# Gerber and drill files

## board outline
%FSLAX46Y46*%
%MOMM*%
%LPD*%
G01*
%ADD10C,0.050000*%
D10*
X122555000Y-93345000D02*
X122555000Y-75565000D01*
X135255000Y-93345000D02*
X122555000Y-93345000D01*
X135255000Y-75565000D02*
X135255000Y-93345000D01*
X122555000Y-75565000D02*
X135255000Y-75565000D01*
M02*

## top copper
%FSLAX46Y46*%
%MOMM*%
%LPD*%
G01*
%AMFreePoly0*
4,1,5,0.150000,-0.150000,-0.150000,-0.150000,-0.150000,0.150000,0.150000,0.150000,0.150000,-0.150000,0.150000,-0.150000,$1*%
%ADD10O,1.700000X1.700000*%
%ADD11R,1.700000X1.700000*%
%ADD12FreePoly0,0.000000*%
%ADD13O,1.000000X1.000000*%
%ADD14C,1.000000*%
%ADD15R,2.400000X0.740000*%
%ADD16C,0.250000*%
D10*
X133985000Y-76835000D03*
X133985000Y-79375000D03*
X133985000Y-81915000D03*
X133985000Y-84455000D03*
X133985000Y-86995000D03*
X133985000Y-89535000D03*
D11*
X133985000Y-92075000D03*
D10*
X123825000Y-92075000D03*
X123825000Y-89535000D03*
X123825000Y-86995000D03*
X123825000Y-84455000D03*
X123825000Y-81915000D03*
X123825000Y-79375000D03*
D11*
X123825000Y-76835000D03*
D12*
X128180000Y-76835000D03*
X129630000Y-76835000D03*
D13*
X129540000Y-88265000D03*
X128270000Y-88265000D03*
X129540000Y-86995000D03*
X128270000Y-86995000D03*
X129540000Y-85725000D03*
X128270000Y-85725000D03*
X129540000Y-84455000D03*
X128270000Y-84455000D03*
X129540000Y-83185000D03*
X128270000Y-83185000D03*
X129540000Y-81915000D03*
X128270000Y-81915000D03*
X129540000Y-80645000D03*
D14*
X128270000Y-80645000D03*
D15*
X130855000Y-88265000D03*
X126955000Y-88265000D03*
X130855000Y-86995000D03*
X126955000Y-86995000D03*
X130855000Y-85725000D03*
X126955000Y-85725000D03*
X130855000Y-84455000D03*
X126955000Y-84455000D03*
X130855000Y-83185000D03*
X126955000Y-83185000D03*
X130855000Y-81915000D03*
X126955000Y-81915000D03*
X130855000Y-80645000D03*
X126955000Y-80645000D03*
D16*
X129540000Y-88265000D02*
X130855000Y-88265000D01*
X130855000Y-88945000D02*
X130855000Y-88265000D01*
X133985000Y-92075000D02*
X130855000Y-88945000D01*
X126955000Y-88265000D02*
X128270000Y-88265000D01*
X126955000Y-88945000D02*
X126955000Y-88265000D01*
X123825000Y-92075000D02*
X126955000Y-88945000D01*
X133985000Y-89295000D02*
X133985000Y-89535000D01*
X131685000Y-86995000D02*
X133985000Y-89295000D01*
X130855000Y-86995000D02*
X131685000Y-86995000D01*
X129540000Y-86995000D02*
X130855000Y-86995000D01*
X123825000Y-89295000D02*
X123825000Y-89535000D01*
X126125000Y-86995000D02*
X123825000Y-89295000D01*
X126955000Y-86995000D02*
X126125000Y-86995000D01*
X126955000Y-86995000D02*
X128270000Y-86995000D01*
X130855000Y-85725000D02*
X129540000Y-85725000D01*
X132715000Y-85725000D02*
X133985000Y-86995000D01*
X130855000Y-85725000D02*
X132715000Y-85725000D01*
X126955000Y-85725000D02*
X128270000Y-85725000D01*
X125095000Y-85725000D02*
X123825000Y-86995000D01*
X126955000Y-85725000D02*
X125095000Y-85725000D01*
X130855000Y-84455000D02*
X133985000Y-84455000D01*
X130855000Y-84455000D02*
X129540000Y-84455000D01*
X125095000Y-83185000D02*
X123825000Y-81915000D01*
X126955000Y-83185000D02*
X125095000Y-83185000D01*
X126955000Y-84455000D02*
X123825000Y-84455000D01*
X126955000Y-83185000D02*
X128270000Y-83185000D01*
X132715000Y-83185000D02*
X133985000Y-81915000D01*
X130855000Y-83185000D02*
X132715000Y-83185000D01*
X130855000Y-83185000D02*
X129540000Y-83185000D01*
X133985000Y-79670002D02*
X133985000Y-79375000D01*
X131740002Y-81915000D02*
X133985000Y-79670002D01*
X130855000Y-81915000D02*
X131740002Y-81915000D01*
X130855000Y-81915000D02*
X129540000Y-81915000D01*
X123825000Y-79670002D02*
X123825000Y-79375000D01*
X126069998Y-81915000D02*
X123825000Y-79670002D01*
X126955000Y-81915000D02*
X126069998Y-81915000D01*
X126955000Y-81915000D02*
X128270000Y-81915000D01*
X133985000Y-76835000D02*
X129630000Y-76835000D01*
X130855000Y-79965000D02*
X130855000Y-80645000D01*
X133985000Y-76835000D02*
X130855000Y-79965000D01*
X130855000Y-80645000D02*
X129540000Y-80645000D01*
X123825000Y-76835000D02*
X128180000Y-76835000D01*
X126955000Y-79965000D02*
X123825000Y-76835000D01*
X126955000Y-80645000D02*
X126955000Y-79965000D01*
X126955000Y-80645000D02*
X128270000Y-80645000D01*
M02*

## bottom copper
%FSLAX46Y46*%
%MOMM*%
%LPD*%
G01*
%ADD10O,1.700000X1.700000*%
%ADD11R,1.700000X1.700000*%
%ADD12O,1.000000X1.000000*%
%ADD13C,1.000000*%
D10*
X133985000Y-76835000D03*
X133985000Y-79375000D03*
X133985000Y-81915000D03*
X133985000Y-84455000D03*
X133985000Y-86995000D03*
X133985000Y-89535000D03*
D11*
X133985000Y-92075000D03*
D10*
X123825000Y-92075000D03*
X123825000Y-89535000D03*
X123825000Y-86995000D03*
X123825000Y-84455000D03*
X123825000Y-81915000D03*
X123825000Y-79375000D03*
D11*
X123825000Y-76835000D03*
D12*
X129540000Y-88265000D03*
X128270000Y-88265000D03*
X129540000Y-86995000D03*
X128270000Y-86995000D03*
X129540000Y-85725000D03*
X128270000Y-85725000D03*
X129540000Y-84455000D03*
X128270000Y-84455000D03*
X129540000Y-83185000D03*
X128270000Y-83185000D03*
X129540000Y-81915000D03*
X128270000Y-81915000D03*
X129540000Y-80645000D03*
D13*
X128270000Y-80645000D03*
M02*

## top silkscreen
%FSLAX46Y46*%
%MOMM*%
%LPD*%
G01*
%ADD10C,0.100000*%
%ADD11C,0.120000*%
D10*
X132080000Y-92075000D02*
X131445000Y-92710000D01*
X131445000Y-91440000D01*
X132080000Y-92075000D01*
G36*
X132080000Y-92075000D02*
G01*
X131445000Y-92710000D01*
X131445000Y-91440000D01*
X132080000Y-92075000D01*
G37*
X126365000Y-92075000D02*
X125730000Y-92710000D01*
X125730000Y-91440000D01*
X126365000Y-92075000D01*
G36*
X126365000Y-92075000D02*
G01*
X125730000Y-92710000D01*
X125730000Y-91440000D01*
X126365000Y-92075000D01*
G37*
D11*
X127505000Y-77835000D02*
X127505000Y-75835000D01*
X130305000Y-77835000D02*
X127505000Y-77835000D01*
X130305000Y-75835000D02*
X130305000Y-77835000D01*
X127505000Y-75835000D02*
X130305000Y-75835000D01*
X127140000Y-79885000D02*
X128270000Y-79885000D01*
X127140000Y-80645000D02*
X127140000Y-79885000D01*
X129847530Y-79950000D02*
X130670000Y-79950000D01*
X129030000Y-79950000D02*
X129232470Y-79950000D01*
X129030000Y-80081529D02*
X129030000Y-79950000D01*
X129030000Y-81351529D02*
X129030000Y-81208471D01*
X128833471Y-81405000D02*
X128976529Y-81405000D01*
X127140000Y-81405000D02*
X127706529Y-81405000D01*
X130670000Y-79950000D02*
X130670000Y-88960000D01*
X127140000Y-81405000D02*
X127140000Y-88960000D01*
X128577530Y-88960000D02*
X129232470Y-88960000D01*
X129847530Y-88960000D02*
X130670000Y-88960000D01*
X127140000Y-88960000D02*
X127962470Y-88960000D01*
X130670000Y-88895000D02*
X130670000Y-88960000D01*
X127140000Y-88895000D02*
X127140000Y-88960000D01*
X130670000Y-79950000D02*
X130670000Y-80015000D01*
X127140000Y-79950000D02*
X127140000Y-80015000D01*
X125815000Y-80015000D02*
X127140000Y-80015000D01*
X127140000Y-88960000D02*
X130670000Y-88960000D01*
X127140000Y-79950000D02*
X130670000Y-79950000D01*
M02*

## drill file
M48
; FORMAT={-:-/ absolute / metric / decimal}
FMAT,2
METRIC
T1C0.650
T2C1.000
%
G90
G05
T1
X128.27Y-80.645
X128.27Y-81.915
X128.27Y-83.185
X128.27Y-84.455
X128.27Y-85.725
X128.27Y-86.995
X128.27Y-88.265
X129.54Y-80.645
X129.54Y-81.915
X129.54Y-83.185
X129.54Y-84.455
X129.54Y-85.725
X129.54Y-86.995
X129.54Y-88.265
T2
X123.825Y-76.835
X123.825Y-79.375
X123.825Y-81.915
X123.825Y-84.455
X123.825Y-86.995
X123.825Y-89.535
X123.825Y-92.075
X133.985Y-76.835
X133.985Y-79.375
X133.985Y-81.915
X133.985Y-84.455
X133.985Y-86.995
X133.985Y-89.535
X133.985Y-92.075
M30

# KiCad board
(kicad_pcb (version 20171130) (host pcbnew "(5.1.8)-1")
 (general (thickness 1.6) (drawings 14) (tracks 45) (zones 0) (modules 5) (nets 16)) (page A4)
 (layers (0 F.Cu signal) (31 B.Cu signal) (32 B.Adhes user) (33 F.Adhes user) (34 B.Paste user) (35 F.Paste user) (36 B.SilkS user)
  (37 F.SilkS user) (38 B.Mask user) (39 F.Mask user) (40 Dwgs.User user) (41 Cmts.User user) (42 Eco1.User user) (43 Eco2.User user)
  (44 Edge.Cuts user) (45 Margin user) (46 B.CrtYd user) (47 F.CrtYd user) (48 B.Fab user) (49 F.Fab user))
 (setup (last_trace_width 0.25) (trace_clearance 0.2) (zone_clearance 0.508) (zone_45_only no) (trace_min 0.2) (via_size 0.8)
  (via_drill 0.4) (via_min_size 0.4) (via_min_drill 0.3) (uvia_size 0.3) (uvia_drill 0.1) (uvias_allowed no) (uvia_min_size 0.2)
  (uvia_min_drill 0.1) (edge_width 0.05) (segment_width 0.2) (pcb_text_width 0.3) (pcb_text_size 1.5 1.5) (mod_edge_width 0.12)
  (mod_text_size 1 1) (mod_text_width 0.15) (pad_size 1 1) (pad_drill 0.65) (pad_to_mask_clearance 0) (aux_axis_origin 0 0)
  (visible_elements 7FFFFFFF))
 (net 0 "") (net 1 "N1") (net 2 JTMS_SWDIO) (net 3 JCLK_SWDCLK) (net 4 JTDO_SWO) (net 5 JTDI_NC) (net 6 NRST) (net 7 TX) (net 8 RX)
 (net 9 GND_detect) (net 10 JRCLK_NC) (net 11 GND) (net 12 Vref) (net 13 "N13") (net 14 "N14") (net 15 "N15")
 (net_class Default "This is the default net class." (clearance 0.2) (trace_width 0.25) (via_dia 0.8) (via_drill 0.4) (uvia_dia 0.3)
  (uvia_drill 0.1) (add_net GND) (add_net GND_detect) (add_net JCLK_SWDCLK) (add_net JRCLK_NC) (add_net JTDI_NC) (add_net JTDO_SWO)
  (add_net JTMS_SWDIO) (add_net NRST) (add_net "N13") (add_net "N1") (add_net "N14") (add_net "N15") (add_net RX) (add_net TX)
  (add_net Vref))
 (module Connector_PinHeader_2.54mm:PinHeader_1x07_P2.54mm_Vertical (layer B.Cu) (at 133.985 92.075)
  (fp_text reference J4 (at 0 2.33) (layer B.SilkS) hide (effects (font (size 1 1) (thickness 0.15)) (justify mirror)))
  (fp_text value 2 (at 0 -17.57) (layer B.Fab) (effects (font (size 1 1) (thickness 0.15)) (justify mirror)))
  (pad 7 thru_hole oval (at 0 -15.24) (size 1.7 1.7) (drill 1) (layers *.Cu *.Mask) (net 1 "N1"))
  (pad 6 thru_hole oval (at 0 -12.7) (size 1.7 1.7) (drill 1) (layers *.Cu *.Mask) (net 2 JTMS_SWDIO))
  (pad 5 thru_hole oval (at 0 -10.16) (size 1.7 1.7) (drill 1) (layers *.Cu *.Mask) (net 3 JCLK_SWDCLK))
  (pad 4 thru_hole oval (at 0 -7.62) (size 1.7 1.7) (drill 1) (layers *.Cu *.Mask) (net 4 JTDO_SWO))
  (pad 3 thru_hole oval (at 0 -5.08) (size 1.7 1.7) (drill 1) (layers *.Cu *.Mask) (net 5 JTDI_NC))
  (pad 2 thru_hole oval (at 0 -2.54) (size 1.7 1.7) (drill 1) (layers *.Cu *.Mask) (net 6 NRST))
  (pad 1 thru_hole rect (at 0 0) (size 1.7 1.7) (drill 1) (layers *.Cu *.Mask) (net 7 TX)))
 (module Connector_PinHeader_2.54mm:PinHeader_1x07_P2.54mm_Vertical (layer B.Cu) (at 123.825 76.835 180)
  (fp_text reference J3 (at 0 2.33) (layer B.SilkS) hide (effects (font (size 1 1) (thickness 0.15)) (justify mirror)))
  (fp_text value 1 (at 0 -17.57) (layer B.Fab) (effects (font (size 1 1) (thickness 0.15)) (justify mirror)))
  (pad 7 thru_hole oval (at 0 -15.24 180) (size 1.7 1.7) (drill 1) (layers *.Cu *.Mask) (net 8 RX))
  (pad 6 thru_hole oval (at 0 -12.7 180) (size 1.7 1.7) (drill 1) (layers *.Cu *.Mask) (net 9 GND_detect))
  (pad 5 thru_hole oval (at 0 -10.16 180) (size 1.7 1.7) (drill 1) (layers *.Cu *.Mask) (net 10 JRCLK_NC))
  (pad 4 thru_hole oval (at 0 -7.62 180) (size 1.7 1.7) (drill 1) (layers *.Cu *.Mask) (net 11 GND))
  (pad 3 thru_hole oval (at 0 -5.08 180) (size 1.7 1.7) (drill 1) (layers *.Cu *.Mask) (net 11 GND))
  (pad 2 thru_hole oval (at 0 -2.54 180) (size 1.7 1.7) (drill 1) (layers *.Cu *.Mask) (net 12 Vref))
  (pad 1 thru_hole rect (at 0 0 180) (size 1.7 1.7) (drill 1) (layers *.Cu *.Mask) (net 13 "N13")))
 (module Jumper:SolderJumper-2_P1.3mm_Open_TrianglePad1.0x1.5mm (layer F.Cu) (at 128.905 76.835)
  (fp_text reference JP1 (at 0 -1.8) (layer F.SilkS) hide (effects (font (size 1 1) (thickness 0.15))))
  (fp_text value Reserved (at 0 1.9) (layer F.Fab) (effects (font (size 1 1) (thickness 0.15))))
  (fp_line (start -1.4 1) (end -1.4 -1) (layer F.SilkS) (width 0.12))
  (fp_line (start 1.4 1) (end -1.4 1) (layer F.SilkS) (width 0.12))
  (fp_line (start 1.4 -1) (end 1.4 1) (layer F.SilkS) (width 0.12))
  (fp_line (start -1.4 -1) (end 1.4 -1) (layer F.SilkS) (width 0.12))
  (pad 1 smd custom (at -0.725 0) (size 0.3 0.3) (layers F.Cu F.Mask) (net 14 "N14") (zone_connect 2)
   (options (clearance outline) (anchor rect)) (primitives))
  (pad 2 smd custom (at 0.725 0) (size 0.3 0.3) (layers F.Cu F.Mask) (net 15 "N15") (zone_connect 2)
   (options (clearance outline) (anchor rect)) (primitives)))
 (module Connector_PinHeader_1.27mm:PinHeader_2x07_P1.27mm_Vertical (layer F.Cu) (at 128.27 80.645)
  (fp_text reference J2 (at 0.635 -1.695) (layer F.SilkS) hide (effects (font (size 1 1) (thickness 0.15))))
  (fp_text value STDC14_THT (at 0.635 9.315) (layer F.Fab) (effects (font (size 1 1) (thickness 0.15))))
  (fp_line (start -1.13 -0.76) (end 0 -0.76) (layer F.SilkS) (width 0.12))
  (fp_line (start -1.13 0) (end -1.13 -0.76) (layer F.SilkS) (width 0.12))
  (fp_line (start 1.57753 -0.695) (end 2.4 -0.695) (layer F.SilkS) (width 0.12))
  (fp_line (start 0.76 -0.695) (end 0.96247 -0.695) (layer F.SilkS) (width 0.12))
  (fp_line (start 0.76 -0.563471) (end 0.76 -0.695) (layer F.SilkS) (width 0.12))
  (fp_line (start 0.76 0.706529) (end 0.76 0.563471) (layer F.SilkS) (width 0.12))
  (fp_line (start 0.563471 0.76) (end 0.706529 0.76) (layer F.SilkS) (width 0.12))
  (fp_line (start -1.13 0.76) (end -0.563471 0.76) (layer F.SilkS) (width 0.12))
  (fp_line (start 2.4 -0.695) (end 2.4 8.315) (layer F.SilkS) (width 0.12))
  (fp_line (start -1.13 0.76) (end -1.13 8.315) (layer F.SilkS) (width 0.12))
  (fp_line (start 0.30753 8.315) (end 0.96247 8.315) (layer F.SilkS) (width 0.12))
  (fp_line (start 1.57753 8.315) (end 2.4 8.315) (layer F.SilkS) (width 0.12))
  (fp_line (start -1.13 8.315) (end -0.30753 8.315) (layer F.SilkS) (width 0.12))
  (pad 14 thru_hole oval (at 1.27 7.62) (size 1 1) (drill 0.65) (layers *.Cu *.Mask) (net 7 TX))
  (pad 13 thru_hole oval (at 0 7.62) (size 1 1) (drill 0.65) (layers *.Cu *.Mask) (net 8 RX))
  (pad 12 thru_hole oval (at 1.27 6.35) (size 1 1) (drill 0.65) (layers *.Cu *.Mask) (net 6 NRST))
  (pad 11 thru_hole oval (at 0 6.35) (size 1 1) (drill 0.65) (layers *.Cu *.Mask) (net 9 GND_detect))
  (pad 10 thru_hole oval (at 1.27 5.08) (size 1 1) (drill 0.65) (layers *.Cu *.Mask) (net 5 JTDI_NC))
  (pad 9 thru_hole oval (at 0 5.08) (size 1 1) (drill 0.65) (layers *.Cu *.Mask) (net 10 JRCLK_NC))
  (pad 8 thru_hole oval (at 1.27 3.81) (size 1 1) (drill 0.65) (layers *.Cu *.Mask) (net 4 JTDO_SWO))
  (pad 7 thru_hole oval (at 0 3.81) (size 1 1) (drill 0.65) (layers *.Cu *.Mask) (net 11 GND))
  (pad 6 thru_hole oval (at 1.27 2.54) (size 1 1) (drill 0.65) (layers *.Cu *.Mask) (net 3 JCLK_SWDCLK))
  (pad 5 thru_hole oval (at 0 2.54) (size 1 1) (drill 0.65) (layers *.Cu *.Mask) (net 11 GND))
  (pad 4 thru_hole oval (at 1.27 1.27) (size 1 1) (drill 0.65) (layers *.Cu *.Mask) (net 2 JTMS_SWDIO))
  (pad 3 thru_hole oval (at 0 1.27) (size 1 1) (drill 0.65) (layers *.Cu *.Mask) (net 12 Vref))
  (pad 2 thru_hole oval (at 1.27 0) (size 1 1) (drill 0.65) (layers *.Cu *.Mask) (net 1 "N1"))
  (pad 1 thru_hole circle (at 0 0) (size 1 1) (drill 0.65) (layers *.Cu *.Mask) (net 13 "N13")))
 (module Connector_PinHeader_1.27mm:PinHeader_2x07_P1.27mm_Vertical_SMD (layer F.Cu) (at 128.905 84.455)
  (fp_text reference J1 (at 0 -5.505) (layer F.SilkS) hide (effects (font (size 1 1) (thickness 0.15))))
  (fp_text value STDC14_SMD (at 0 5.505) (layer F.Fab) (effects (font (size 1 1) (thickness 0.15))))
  (fp_line (start 1.765 4.44) (end 1.765 4.505) (layer F.SilkS) (width 0.12))
  (fp_line (start -1.765 4.44) (end -1.765 4.505) (layer F.SilkS) (width 0.12))
  (fp_line (start 1.765 -4.505) (end 1.765 -4.44) (layer F.SilkS) (width 0.12))
  (fp_line (start -1.765 -4.505) (end -1.765 -4.44) (layer F.SilkS) (width 0.12))
  (fp_line (start -3.09 -4.44) (end -1.765 -4.44) (layer F.SilkS) (width 0.12))
  (fp_line (start -1.765 4.505) (end 1.765 4.505) (layer F.SilkS) (width 0.12))
  (fp_line (start -1.765 -4.505) (end 1.765 -4.505) (layer F.SilkS) (width 0.12))
  (pad 14 smd rect (at 1.95 3.81) (size 2.4 0.74) (layers F.Cu F.Paste F.Mask) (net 7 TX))
  (pad 13 smd rect (at -1.95 3.81) (size 2.4 0.74) (layers F.Cu F.Paste F.Mask) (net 8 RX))
  (pad 12 smd rect (at 1.95 2.54) (size 2.4 0.74) (layers F.Cu F.Paste F.Mask) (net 6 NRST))
  (pad 11 smd rect (at -1.95 2.54) (size 2.4 0.74) (layers F.Cu F.Paste F.Mask) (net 9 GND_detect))
  (pad 10 smd rect (at 1.95 1.27) (size 2.4 0.74) (layers F.Cu F.Paste F.Mask) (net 5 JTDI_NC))
  (pad 9 smd rect (at -1.95 1.27) (size 2.4 0.74) (layers F.Cu F.Paste F.Mask) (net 10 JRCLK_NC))
  (pad 8 smd rect (at 1.95 0) (size 2.4 0.74) (layers F.Cu F.Paste F.Mask) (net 4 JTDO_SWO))
  (pad 7 smd rect (at -1.95 0) (size 2.4 0.74) (layers F.Cu F.Paste F.Mask) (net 11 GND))
  (pad 6 smd rect (at 1.95 -1.27) (size 2.4 0.74) (layers F.Cu F.Paste F.Mask) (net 3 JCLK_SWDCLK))
  (pad 5 smd rect (at -1.95 -1.27) (size 2.4 0.74) (layers F.Cu F.Paste F.Mask) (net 11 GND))
  (pad 4 smd rect (at 1.95 -2.54) (size 2.4 0.74) (layers F.Cu F.Paste F.Mask) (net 2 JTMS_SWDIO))
  (pad 3 smd rect (at -1.95 -2.54) (size 2.4 0.74) (layers F.Cu F.Paste F.Mask) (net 12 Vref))
  (pad 2 smd rect (at 1.95 -3.81) (size 2.4 0.74) (layers F.Cu F.Paste F.Mask) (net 1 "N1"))
  (pad 1 smd rect (at -1.95 -3.81) (size 2.4 0.74) (layers F.Cu F.Paste F.Mask) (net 13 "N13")))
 (gr_line (start 122.555 93.345) (end 122.555 75.565) (layer Edge.Cuts) (width 0.05))
 (gr_line (start 135.255 93.345) (end 122.555 93.345) (layer Edge.Cuts) (width 0.05))
 (gr_line (start 135.255 75.565) (end 135.255 93.345) (layer Edge.Cuts) (width 0.05))
 (gr_line (start 122.555 75.565) (end 135.255 75.565) (layer Edge.Cuts) (width 0.05))
 (gr_poly (pts (xy 132.08 92.075) (xy 131.445 92.71) (xy 131.445 91.44)) (layer F.SilkS) (width 0.1))
 (gr_poly (pts (xy 126.365 92.075) (xy 125.73 92.71) (xy 125.73 91.44)) (layer F.SilkS) (width 0.1))
 (segment (start 129.54 88.265) (end 130.855 88.265) (width 0.25) (layer F.Cu) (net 7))
 (segment (start 130.855 88.945) (end 130.855 88.265) (width 0.25) (layer F.Cu) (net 7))
 (segment (start 133.985 92.075) (end 130.855 88.945) (width 0.25) (layer F.Cu) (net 7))
 (segment (start 126.955 88.265) (end 128.27 88.265) (width 0.25) (layer F.Cu) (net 8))
 (segment (start 126.955 88.945) (end 126.955 88.265) (width 0.25) (layer F.Cu) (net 8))
 (segment (start 123.825 92.075) (end 126.955 88.945) (width 0.25) (layer F.Cu) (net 8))
 (segment (start 133.985 89.295) (end 133.985 89.535) (width 0.25) (layer F.Cu) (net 6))
 (segment (start 131.685 86.995) (end 133.985 89.295) (width 0.25) (layer F.Cu) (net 6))
 (segment (start 130.855 86.995) (end 131.685 86.995) (width 0.25) (layer F.Cu) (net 6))
 (segment (start 129.54 86.995) (end 130.855 86.995) (width 0.25) (layer F.Cu) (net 6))
 (segment (start 123.825 89.295) (end 123.825 89.535) (width 0.25) (layer F.Cu) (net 9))
 (segment (start 126.125 86.995) (end 123.825 89.295) (width 0.25) (layer F.Cu) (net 9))
 (segment (start 126.955 86.995) (end 126.125 86.995) (width 0.25) (layer F.Cu) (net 9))
 (segment (start 126.955 86.995) (end 128.27 86.995) (width 0.25) (layer F.Cu) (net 9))
 (segment (start 130.855 85.725) (end 129.54 85.725) (width 0.25) (layer F.Cu) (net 5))
 (segment (start 132.715 85.725) (end 133.985 86.995) (width 0.25) (layer F.Cu) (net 5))
 (segment (start 130.855 85.725) (end 132.715 85.725) (width 0.25) (layer F.Cu) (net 5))
 (segment (start 126.955 85.725) (end 128.27 85.725) (width 0.25) (layer F.Cu) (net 10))
 (segment (start 125.095 85.725) (end 123.825 86.995) (width 0.25) (layer F.Cu) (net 10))
 (segment (start 126.955 85.725) (end 125.095 85.725) (width 0.25) (layer F.Cu) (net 10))
 (segment (start 130.855 84.455) (end 133.985 84.455) (width 0.25) (layer F.Cu) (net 4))
 (segment (start 130.855 84.455) (end 129.54 84.455) (width 0.25) (layer F.Cu) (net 4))
 (segment (start 125.095 83.185) (end 123.825 81.915) (width 0.25) (layer F.Cu) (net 11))
 (segment (start 126.955 83.185) (end 125.095 83.185) (width 0.25) (layer F.Cu) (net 11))
 (segment (start 126.955 84.455) (end 123.825 84.455) (width 0.25) (layer F.Cu) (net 11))
 (segment (start 126.955 83.185) (end 128.27 83.185) (width 0.25) (layer F.Cu) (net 11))
 (segment (start 132.715 83.185) (end 133.985 81.915) (width 0.25) (layer F.Cu) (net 3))
 (segment (start 130.855 83.185) (end 132.715 83.185) (width 0.25) (layer F.Cu) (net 3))
 (segment (start 130.855 83.185) (end 129.54 83.185) (width 0.25) (layer F.Cu) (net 3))
 (segment (start 133.985 79.670002) (end 133.985 79.375) (width 0.25) (layer F.Cu) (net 2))
 (segment (start 131.740002 81.915) (end 133.985 79.670002) (width 0.25) (layer F.Cu) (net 2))
 (segment (start 130.855 81.915) (end 131.740002 81.915) (width 0.25) (layer F.Cu) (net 2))
 (segment (start 130.855 81.915) (end 129.54 81.915) (width 0.25) (layer F.Cu) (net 2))
 (segment (start 123.825 79.670002) (end 123.825 79.375) (width 0.25) (layer F.Cu) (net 12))
 (segment (start 126.069998 81.915) (end 123.825 79.670002) (width 0.25) (layer F.Cu) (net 12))
 (segment (start 126.955 81.915) (end 126.069998 81.915) (width 0.25) (layer F.Cu) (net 12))
 (segment (start 126.955 81.915) (end 128.27 81.915) (width 0.25) (layer F.Cu) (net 12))
 (segment (start 133.985 76.835) (end 129.63 76.835) (width 0.25) (layer F.Cu) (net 1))
 (segment (start 130.855 79.965) (end 130.855 80.645) (width 0.25) (layer F.Cu) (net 1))
 (segment (start 133.985 76.835) (end 130.855 79.965) (width 0.25) (layer F.Cu) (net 1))
 (segment (start 130.855 80.645) (end 129.54 80.645) (width 0.25) (layer F.Cu) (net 1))
 (segment (start 123.825 76.835) (end 128.18 76.835) (width 0.25) (layer F.Cu) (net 13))
 (segment (start 126.955 79.965) (end 123.825 76.835) (width 0.25) (layer F.Cu) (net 13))
 (segment (start 126.955 80.645) (end 126.955 79.965) (width 0.25) (layer F.Cu) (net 13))
 (segment (start 126.955 80.645) (end 128.27 80.645) (width 0.25) (layer F.Cu) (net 13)))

